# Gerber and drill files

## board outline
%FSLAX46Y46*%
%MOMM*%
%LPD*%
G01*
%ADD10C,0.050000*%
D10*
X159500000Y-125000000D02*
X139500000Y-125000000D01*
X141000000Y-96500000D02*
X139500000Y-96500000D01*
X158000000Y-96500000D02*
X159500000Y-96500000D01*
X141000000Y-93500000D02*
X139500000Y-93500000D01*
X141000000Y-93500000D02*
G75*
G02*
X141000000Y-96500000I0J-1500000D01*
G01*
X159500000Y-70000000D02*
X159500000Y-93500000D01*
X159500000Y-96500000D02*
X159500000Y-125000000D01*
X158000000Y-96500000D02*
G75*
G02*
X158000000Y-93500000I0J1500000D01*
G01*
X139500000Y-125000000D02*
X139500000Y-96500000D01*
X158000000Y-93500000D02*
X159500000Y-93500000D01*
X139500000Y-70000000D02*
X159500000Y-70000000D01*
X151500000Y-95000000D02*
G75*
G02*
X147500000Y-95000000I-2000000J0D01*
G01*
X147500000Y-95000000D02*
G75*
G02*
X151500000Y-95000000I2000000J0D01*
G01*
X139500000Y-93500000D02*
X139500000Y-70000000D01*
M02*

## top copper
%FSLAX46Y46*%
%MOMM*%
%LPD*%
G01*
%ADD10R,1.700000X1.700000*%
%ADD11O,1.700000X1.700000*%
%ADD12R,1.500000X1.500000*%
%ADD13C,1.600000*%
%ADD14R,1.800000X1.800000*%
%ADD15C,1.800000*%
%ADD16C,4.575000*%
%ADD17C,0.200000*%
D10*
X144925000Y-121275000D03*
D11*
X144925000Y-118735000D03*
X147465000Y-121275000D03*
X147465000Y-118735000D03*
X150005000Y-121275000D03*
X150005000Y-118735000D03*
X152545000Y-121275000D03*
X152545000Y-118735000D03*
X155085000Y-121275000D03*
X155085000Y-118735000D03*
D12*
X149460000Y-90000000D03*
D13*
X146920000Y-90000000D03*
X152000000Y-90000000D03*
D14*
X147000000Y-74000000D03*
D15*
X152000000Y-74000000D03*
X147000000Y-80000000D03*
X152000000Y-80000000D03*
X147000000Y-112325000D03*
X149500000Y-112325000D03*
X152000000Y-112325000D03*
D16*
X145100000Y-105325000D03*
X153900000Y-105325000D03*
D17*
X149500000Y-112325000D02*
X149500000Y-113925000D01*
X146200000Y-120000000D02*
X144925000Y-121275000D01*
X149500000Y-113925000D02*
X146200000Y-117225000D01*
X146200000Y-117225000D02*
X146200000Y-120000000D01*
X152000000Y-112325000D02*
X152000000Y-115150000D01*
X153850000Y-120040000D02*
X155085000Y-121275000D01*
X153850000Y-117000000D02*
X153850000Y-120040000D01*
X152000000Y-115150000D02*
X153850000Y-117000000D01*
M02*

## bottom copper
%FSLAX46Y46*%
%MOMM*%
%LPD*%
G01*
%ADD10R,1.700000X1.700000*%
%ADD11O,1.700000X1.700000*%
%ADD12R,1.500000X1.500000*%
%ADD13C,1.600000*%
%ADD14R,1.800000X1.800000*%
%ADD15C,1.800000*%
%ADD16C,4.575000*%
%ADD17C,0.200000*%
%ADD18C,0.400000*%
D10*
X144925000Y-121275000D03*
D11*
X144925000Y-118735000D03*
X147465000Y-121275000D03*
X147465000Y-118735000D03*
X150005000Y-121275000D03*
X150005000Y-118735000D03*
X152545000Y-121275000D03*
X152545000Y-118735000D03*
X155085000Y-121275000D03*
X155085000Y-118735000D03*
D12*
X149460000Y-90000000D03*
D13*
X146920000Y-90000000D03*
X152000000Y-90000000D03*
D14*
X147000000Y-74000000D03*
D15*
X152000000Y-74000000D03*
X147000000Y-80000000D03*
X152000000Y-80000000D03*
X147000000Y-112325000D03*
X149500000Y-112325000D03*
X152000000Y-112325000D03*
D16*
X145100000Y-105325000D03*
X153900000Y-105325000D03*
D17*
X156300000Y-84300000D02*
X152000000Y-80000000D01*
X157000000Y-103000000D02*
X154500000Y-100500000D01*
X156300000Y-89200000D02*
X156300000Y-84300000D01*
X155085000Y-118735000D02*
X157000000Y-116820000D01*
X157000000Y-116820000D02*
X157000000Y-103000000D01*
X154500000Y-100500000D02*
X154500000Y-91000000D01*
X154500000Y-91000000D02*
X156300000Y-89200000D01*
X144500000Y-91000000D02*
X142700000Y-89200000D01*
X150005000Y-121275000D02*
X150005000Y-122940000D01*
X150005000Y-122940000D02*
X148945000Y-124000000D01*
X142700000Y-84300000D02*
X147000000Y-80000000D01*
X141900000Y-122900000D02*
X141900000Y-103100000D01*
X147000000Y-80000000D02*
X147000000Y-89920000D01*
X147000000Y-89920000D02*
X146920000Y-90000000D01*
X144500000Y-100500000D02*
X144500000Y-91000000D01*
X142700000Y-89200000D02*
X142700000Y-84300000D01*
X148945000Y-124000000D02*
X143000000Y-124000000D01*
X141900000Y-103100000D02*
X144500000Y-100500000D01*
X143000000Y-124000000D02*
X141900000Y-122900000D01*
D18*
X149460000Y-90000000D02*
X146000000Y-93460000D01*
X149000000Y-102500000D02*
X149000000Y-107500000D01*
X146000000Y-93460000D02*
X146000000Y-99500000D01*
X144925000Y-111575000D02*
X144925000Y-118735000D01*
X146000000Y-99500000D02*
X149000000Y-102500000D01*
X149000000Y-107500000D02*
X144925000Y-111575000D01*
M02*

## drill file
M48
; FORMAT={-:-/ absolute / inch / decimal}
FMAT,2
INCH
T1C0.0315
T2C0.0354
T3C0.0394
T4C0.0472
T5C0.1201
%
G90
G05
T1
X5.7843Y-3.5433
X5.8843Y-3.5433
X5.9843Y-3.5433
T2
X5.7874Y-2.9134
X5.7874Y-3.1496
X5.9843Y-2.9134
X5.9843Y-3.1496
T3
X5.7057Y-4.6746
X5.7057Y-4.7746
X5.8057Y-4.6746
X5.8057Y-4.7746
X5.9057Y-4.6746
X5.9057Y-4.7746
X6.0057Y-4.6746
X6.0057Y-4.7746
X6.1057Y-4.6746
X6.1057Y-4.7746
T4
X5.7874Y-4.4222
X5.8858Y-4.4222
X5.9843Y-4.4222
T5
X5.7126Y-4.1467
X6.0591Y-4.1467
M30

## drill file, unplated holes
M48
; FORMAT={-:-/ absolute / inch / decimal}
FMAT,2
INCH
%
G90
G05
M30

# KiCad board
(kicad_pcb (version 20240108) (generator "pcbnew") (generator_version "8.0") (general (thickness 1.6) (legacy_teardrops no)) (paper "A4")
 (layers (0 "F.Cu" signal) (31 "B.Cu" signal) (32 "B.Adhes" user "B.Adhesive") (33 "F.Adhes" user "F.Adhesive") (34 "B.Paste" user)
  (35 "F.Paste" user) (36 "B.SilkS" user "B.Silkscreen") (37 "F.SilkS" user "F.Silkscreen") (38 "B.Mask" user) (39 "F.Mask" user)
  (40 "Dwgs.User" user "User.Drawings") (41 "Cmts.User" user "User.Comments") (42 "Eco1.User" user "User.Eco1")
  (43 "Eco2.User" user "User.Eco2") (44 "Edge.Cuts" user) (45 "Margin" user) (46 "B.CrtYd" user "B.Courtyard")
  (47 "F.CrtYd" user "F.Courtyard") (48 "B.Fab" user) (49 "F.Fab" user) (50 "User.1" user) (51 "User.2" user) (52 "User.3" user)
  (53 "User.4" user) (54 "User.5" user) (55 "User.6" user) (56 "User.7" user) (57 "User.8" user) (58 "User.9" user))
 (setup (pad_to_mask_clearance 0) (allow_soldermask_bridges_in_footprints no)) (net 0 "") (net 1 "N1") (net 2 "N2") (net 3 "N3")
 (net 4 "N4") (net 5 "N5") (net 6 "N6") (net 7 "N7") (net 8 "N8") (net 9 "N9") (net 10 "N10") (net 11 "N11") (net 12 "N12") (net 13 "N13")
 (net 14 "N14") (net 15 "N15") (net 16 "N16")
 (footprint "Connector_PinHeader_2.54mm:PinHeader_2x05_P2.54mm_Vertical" (layer "F.Cu") (at 144.925 121.275 90)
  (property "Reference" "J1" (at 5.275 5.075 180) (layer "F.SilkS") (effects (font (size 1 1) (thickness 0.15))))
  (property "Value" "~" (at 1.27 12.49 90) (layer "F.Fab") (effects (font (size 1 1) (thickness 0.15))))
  (pad "1" thru_hole rect (at 0 0 90) (size 1.7 1.7) (drill 1) (layers "*.Cu" "*.Mask") (remove_unused_layers no) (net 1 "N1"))
  (pad "2" thru_hole oval (at 2.54 0 90) (size 1.7 1.7) (drill 1) (layers "*.Cu" "*.Mask") (remove_unused_layers no) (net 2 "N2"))
  (pad "3" thru_hole oval (at 0 2.54 90) (size 1.7 1.7) (drill 1) (layers "*.Cu" "*.Mask") (remove_unused_layers no) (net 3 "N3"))
  (pad "4" thru_hole oval (at 2.54 2.54 90) (size 1.7 1.7) (drill 1) (layers "*.Cu" "*.Mask") (remove_unused_layers no) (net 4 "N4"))
  (pad "5" thru_hole oval (at 0 5.08 90) (size 1.7 1.7) (drill 1) (layers "*.Cu" "*.Mask") (remove_unused_layers no) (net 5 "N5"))
  (pad "6" thru_hole oval (at 2.54 5.08 90) (size 1.7 1.7) (drill 1) (layers "*.Cu" "*.Mask") (remove_unused_layers no) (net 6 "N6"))
  (pad "7" thru_hole oval (at 0 7.62 90) (size 1.7 1.7) (drill 1) (layers "*.Cu" "*.Mask") (remove_unused_layers no) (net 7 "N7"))
  (pad "8" thru_hole oval (at 2.54 7.62 90) (size 1.7 1.7) (drill 1) (layers "*.Cu" "*.Mask") (remove_unused_layers no) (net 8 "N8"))
  (pad "9" thru_hole oval (at 0 10.16 90) (size 1.7 1.7) (drill 1) (layers "*.Cu" "*.Mask") (remove_unused_layers no) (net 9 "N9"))
  (pad "10" thru_hole oval (at 2.54 10.16 90) (size 1.7 1.7) (drill 1) (layers "*.Cu" "*.Mask") (remove_unused_layers no) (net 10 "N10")))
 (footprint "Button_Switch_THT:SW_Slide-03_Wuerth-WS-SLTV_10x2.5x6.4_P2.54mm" (layer "F.Cu") (at 149.46 90)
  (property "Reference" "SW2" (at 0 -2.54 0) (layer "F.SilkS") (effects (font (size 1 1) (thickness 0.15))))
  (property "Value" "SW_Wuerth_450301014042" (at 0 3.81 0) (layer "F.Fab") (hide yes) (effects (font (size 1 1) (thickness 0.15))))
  (pad "1" thru_hole rect (at 0 0) (size 1.5 1.5) (drill 0.8) (layers "*.Cu" "*.Mask") (remove_unused_layers no) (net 2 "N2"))
  (pad "2" thru_hole circle (at -2.54 0) (size 1.6 1.6) (drill 0.8) (layers "*.Cu" "*.Mask") (remove_unused_layers no) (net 5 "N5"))
  (pad "3" thru_hole circle (at 2.54 0) (size 1.6 1.6) (drill 0.8) (layers "*.Cu" "*.Mask") (remove_unused_layers no) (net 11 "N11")))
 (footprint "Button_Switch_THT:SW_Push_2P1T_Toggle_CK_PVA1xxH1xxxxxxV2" (layer "F.Cu") (at 147 74)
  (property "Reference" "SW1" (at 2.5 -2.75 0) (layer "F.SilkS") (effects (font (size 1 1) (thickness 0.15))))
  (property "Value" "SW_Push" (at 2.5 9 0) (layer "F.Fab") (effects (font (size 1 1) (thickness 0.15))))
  (pad "1" thru_hole rect (at 0 0) (size 1.8 1.8) (drill 0.9) (layers "*.Cu" "*.Mask") (remove_unused_layers no) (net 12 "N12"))
  (pad "2" thru_hole circle (at 5 0) (size 1.8 1.8) (drill 0.9) (layers "*.Cu" "*.Mask") (remove_unused_layers no) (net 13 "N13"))
  (pad "3" thru_hole circle (at 0 6) (size 1.8 1.8) (drill 0.9) (layers "*.Cu" "*.Mask") (remove_unused_layers no) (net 5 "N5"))
  (pad "4" thru_hole circle (at 5 6) (size 1.8 1.8) (drill 0.9) (layers "*.Cu" "*.Mask") (remove_unused_layers no) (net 10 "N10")))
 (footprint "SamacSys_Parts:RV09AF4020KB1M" (layer "F.Cu") (at 147 112.325)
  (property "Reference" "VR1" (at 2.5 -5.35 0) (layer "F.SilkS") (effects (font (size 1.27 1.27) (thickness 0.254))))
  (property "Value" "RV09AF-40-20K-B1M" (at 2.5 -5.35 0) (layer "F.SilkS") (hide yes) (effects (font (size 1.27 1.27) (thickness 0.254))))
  (pad "1" thru_hole circle (at 0 0 90) (size 1.8 1.8) (drill 1.2) (layers "*.Cu" "*.Mask" "F.SilkS") (remove_unused_layers no)
   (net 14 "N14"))
  (pad "2" thru_hole circle (at 2.5 0 90) (size 1.8 1.8) (drill 1.2) (layers "*.Cu" "*.Mask" "F.SilkS") (remove_unused_layers no)
   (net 1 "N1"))
  (pad "3" thru_hole circle (at 5 0 90) (size 1.8 1.8) (drill 1.2) (layers "*.Cu" "*.Mask" "F.SilkS") (remove_unused_layers no) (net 9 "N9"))
  (pad "MH1" thru_hole circle (at -1.9 -7 90) (size 4.575 4.575) (drill 3.05) (layers "*.Cu" "*.Mask" "F.SilkS") (remove_unused_layers no)
   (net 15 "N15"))
  (pad "MH2" thru_hole circle (at 6.9 -7 90) (size 4.575 4.575) (drill 3.05) (layers "*.Cu" "*.Mask" "F.SilkS") (remove_unused_layers no)
   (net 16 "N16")))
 (gr_line (start 159.5 125) (end 139.5 125) (stroke (width 0.05) (type default)) (layer "Edge.Cuts"))
 (gr_line (start 141 96.5) (end 139.5 96.5) (stroke (width 0.05) (type default)) (layer "Edge.Cuts"))
 (gr_line (start 158 96.5) (end 159.5 96.5) (stroke (width 0.05) (type default)) (layer "Edge.Cuts"))
 (gr_line (start 141 93.5) (end 139.5 93.5) (stroke (width 0.05) (type default)) (layer "Edge.Cuts"))
 (gr_arc (start 141 93.5) (mid 142.5 95) (end 141 96.5) (stroke (width 0.05) (type default)) (layer "Edge.Cuts"))
 (gr_line (start 159.5 70) (end 159.5 93.5) (stroke (width 0.05) (type default)) (layer "Edge.Cuts"))
 (gr_line (start 159.5 96.5) (end 159.5 125) (stroke (width 0.05) (type default)) (layer "Edge.Cuts"))
 (gr_arc (start 158 96.5) (mid 156.5 95) (end 158 93.5) (stroke (width 0.05) (type default)) (layer "Edge.Cuts"))
 (gr_line (start 139.5 125) (end 139.5 96.5) (stroke (width 0.05) (type default)) (layer "Edge.Cuts"))
 (gr_line (start 158 93.5) (end 159.5 93.5) (stroke (width 0.05) (type default)) (layer "Edge.Cuts"))
 (gr_line (start 139.5 70) (end 159.5 70) (stroke (width 0.05) (type default)) (layer "Edge.Cuts"))
 (gr_circle (center 149.5 95) (end 149.5 97) (stroke (width 0.05) (type default)) (fill none) (layer "Edge.Cuts"))
 (gr_line (start 139.5 93.5) (end 139.5 70) (stroke (width 0.05) (type default)) (layer "Edge.Cuts"))
 (segment (start 156.3 84.3) (end 152 80) (width 0.2) (layer "B.Cu") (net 10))
 (segment (start 157 103) (end 154.5 100.5) (width 0.2) (layer "B.Cu") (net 10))
 (segment (start 156.3 89.2) (end 156.3 84.3) (width 0.2) (layer "B.Cu") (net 10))
 (segment (start 155.085 118.735) (end 157 116.82) (width 0.2) (layer "B.Cu") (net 10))
 (segment (start 157 116.82) (end 157 103) (width 0.2) (layer "B.Cu") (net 10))
 (segment (start 154.5 100.5) (end 154.5 91) (width 0.2) (layer "B.Cu") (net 10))
 (segment (start 154.5 91) (end 156.3 89.2) (width 0.2) (layer "B.Cu") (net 10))
 (segment (start 144.5 91) (end 142.7 89.2) (width 0.2) (layer "B.Cu") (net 5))
 (segment (start 150.005 121.275) (end 150.005 122.94) (width 0.2) (layer "B.Cu") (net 5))
 (segment (start 150.005 122.94) (end 148.945 124) (width 0.2) (layer "B.Cu") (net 5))
 (segment (start 142.7 84.3) (end 147 80) (width 0.2) (layer "B.Cu") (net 5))
 (segment (start 141.9 122.9) (end 141.9 103.1) (width 0.2) (layer "B.Cu") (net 5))
 (segment (start 147 80) (end 147 89.92) (width 0.2) (layer "B.Cu") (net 5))
 (segment (start 147 89.92) (end 146.92 90) (width 0.2) (layer "B.Cu") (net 5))
 (segment (start 144.5 100.5) (end 144.5 91) (width 0.2) (layer "B.Cu") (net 5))
 (segment (start 142.7 89.2) (end 142.7 84.3) (width 0.2) (layer "B.Cu") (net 5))
 (segment (start 148.945 124) (end 143 124) (width 0.2) (layer "B.Cu") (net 5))
 (segment (start 141.9 103.1) (end 144.5 100.5) (width 0.2) (layer "B.Cu") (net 5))
 (segment (start 143 124) (end 141.9 122.9) (width 0.2) (layer "B.Cu") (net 5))
 (segment (start 149.46 90) (end 146 93.46) (width 0.4) (layer "B.Cu") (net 2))
 (segment (start 149 102.5) (end 149 107.5) (width 0.4) (layer "B.Cu") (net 2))
 (segment (start 146 93.46) (end 146 99.5) (width 0.4) (layer "B.Cu") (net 2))
 (segment (start 144.925 111.575) (end 144.925 118.735) (width 0.4) (layer "B.Cu") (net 2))
 (segment (start 146 99.5) (end 149 102.5) (width 0.4) (layer "B.Cu") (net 2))
 (segment (start 149 107.5) (end 144.925 111.575) (width 0.4) (layer "B.Cu") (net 2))
 (segment (start 149.5 112.325) (end 149.5 113.925) (width 0.2) (layer "F.Cu") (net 1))
 (segment (start 146.2 120) (end 144.925 121.275) (width 0.2) (layer "F.Cu") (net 1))
 (segment (start 149.5 113.925) (end 146.2 117.225) (width 0.2) (layer "F.Cu") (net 1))
 (segment (start 146.2 117.225) (end 146.2 120) (width 0.2) (layer "F.Cu") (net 1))
 (segment (start 152 112.325) (end 152 115.15) (width 0.2) (layer "F.Cu") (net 9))
 (segment (start 153.85 120.04) (end 155.085 121.275) (width 0.2) (layer "F.Cu") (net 9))
 (segment (start 153.85 117) (end 153.85 120.04) (width 0.2) (layer "F.Cu") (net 9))
 (segment (start 152 115.15) (end 153.85 117) (width 0.2) (layer "F.Cu") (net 9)))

